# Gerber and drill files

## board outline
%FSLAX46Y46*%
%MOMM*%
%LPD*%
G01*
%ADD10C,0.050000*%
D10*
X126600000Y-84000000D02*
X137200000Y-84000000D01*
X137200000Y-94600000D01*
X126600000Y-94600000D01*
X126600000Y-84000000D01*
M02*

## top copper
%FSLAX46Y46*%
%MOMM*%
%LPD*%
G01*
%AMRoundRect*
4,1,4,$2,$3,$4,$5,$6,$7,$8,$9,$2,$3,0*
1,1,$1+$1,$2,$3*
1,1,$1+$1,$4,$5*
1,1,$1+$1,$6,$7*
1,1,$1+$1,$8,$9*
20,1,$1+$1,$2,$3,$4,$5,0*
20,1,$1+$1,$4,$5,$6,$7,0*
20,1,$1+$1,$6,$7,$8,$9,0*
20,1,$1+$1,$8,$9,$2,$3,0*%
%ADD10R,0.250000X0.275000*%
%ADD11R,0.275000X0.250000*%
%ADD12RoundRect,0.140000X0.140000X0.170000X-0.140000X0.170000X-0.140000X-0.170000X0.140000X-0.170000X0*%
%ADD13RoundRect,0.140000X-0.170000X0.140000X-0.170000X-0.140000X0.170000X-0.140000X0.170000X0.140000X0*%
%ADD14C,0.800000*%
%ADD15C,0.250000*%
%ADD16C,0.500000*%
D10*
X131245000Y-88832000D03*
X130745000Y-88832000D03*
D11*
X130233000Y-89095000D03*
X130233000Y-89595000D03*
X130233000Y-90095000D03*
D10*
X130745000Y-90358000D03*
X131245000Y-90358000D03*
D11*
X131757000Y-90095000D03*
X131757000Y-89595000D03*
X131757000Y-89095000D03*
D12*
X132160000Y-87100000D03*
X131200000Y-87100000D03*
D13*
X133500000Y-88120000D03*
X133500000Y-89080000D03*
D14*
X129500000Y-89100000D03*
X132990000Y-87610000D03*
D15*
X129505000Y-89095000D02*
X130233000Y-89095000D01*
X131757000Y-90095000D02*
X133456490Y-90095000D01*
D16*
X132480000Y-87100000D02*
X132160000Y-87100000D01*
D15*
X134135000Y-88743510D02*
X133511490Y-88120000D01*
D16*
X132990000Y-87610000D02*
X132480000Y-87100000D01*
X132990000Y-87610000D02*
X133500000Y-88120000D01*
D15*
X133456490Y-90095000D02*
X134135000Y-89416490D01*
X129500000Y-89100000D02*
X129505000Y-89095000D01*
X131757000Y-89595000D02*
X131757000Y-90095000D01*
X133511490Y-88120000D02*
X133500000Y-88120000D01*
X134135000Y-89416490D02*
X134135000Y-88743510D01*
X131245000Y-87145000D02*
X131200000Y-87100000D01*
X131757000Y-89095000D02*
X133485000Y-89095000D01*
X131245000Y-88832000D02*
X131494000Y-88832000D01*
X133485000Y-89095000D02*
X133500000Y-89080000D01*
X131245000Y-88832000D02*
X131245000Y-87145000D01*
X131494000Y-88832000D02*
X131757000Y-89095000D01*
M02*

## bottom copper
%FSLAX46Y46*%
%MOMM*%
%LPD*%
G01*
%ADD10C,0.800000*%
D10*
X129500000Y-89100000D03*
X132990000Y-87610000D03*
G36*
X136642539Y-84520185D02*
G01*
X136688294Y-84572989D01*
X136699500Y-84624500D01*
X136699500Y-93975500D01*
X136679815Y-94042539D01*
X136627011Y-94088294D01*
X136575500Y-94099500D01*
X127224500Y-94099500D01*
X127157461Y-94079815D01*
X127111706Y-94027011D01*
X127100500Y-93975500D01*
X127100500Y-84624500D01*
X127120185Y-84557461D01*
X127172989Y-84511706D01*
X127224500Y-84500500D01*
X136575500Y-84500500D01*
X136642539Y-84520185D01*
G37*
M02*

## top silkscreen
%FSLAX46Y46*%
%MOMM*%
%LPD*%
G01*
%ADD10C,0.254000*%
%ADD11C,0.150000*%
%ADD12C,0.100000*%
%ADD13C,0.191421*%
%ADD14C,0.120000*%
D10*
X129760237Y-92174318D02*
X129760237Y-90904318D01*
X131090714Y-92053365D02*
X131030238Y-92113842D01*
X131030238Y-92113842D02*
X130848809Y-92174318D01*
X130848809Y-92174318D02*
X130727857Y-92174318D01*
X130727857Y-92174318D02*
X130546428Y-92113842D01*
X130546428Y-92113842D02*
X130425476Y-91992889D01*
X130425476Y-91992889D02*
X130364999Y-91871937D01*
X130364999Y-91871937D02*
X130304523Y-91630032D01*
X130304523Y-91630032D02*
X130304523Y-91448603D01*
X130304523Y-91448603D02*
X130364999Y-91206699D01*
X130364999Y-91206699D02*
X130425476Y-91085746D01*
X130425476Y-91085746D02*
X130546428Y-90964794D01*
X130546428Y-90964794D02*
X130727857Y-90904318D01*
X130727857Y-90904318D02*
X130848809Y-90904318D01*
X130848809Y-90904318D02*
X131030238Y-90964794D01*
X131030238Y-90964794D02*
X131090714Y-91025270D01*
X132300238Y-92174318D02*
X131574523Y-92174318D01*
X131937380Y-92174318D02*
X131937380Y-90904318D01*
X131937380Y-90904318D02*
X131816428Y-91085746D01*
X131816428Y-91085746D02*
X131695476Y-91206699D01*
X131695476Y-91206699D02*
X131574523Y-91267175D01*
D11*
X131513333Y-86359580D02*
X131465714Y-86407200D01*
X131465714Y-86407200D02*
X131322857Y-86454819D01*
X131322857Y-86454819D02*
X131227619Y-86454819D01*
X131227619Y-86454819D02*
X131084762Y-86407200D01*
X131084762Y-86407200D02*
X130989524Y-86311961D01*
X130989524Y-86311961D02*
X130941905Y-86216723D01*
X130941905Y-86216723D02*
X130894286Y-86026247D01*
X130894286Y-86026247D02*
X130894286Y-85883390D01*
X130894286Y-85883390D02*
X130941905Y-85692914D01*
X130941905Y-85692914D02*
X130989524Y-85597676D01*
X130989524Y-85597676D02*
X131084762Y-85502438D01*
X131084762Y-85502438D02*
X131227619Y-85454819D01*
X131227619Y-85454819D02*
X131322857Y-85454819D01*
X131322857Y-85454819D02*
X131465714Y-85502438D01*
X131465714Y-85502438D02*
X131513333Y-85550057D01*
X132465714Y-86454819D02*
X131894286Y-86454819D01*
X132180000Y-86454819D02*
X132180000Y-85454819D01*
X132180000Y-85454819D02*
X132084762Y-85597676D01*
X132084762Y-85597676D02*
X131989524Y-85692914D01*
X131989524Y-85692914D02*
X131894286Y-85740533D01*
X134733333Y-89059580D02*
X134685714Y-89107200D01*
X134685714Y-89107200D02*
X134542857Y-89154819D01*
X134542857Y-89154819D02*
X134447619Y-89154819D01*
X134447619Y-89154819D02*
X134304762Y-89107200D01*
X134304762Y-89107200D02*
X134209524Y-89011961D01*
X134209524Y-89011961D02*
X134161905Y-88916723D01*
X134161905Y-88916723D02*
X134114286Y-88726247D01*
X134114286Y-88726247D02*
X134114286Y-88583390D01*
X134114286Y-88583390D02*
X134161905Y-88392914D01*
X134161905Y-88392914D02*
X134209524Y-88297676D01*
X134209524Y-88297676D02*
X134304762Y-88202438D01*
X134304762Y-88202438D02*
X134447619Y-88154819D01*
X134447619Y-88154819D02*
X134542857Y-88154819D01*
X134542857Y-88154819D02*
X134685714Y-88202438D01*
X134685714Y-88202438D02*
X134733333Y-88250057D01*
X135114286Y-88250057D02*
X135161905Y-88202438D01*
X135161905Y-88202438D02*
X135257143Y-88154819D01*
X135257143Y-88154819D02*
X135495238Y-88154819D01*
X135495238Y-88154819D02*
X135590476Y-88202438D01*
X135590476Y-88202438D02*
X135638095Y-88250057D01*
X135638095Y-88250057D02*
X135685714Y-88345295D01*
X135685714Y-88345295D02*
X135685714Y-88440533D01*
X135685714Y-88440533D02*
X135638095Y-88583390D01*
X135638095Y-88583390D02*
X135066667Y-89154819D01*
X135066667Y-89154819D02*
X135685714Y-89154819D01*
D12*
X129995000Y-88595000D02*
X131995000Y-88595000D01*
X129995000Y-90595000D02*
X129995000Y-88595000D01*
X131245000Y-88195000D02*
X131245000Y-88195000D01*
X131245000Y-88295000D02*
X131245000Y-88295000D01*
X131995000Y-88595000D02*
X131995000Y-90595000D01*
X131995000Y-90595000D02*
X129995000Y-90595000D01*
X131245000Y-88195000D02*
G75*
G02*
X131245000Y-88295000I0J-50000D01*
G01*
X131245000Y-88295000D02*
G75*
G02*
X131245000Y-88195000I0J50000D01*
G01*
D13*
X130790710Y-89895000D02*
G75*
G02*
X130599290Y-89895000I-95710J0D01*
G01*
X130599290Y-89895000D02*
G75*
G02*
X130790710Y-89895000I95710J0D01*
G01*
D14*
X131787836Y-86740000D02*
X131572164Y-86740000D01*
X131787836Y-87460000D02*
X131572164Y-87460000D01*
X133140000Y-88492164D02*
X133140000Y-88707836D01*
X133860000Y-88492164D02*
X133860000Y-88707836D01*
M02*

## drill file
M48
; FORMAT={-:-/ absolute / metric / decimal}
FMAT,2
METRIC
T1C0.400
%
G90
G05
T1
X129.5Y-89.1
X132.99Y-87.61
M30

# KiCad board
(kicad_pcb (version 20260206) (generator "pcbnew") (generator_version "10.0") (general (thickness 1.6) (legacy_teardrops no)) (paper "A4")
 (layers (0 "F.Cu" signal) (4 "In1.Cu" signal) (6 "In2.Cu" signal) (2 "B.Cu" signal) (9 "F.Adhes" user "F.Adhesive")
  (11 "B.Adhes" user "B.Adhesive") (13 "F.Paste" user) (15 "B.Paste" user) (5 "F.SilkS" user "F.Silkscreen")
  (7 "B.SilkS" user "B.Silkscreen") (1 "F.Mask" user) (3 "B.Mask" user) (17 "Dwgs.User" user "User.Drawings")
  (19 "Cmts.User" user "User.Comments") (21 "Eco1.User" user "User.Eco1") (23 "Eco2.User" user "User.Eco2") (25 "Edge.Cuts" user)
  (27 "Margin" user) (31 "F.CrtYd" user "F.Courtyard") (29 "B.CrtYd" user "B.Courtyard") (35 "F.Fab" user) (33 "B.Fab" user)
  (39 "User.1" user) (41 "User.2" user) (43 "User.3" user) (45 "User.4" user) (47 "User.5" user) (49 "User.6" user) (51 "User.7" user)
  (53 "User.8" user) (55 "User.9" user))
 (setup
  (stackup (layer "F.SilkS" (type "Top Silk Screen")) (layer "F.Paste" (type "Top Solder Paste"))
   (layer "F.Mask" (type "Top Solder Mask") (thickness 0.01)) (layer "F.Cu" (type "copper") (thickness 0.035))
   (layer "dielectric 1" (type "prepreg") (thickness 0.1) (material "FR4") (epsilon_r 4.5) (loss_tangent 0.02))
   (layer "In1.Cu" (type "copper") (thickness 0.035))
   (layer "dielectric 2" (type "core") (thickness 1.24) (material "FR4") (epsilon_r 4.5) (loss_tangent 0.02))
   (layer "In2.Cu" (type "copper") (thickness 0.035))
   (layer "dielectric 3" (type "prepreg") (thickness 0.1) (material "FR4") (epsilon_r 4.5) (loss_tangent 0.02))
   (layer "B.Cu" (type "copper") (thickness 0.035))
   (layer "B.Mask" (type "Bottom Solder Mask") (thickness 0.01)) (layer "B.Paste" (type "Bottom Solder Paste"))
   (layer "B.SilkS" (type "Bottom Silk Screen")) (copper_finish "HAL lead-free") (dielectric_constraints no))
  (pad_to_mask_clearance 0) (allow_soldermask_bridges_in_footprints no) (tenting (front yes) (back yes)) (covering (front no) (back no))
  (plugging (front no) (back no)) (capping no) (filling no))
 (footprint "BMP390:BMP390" (layer "F.Cu") (at 130.995 89.595)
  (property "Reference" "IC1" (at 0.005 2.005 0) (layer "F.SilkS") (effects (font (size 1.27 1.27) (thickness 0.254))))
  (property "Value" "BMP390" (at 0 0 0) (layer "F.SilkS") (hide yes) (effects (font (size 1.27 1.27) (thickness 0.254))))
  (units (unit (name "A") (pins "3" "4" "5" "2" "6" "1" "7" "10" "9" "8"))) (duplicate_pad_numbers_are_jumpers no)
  (fp_line (start -1 -1) (end 1 -1) (stroke (width 0.1) (type solid)) (layer "F.SilkS"))
  (fp_line (start -1 1) (end -1 -1) (stroke (width 0.1) (type solid)) (layer "F.SilkS"))
  (fp_line (start 0.25 -1.4) (end 0.25 -1.4) (stroke (width 0.1) (type solid)) (layer "F.SilkS"))
  (fp_line (start 0.25 -1.3) (end 0.25 -1.3) (stroke (width 0.1) (type solid)) (layer "F.SilkS"))
  (fp_line (start 1 -1) (end 1 1) (stroke (width 0.1) (type solid)) (layer "F.SilkS"))
  (fp_line (start 1 1) (end -1 1) (stroke (width 0.1) (type solid)) (layer "F.SilkS"))
  (fp_arc (start 0.25 -1.4) (mid 0.3 -1.35) (end 0.25 -1.3) (stroke (width 0.1) (type solid)) (layer "F.SilkS"))
  (fp_arc (start 0.25 -1.3) (mid 0.2 -1.35) (end 0.25 -1.4) (stroke (width 0.1) (type solid)) (layer "F.SilkS"))
  (fp_circle (center -0.3 0.3) (end -0.4 0.2) (stroke (width 0.1) (type solid)) (fill yes) (layer "F.SilkS"))
  (pad "1" smd rect (at 0.25 -0.763) (size 0.25 0.275) (layers "F.Cu" "F.Mask" "F.Paste") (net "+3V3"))
  (pad "2" smd rect (at -0.25 -0.763) (size 0.25 0.275) (layers "F.Cu" "F.Mask" "F.Paste") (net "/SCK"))
  (pad "3" smd rect (at -0.762 -0.5 90) (size 0.25 0.275) (layers "F.Cu" "F.Mask" "F.Paste") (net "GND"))
  (pad "4" smd rect (at -0.762 0 90) (size 0.25 0.275) (layers "F.Cu" "F.Mask" "F.Paste") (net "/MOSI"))
  (pad "5" smd rect (at -0.762 0.5 90) (size 0.25 0.275) (layers "F.Cu" "F.Mask" "F.Paste") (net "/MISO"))
  (pad "6" smd rect (at -0.25 0.763) (size 0.25 0.275) (layers "F.Cu" "F.Mask" "F.Paste") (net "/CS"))
  (pad "7" smd rect (at 0.25 0.763) (size 0.25 0.275) (layers "F.Cu" "F.Mask" "F.Paste") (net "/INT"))
  (pad "8" smd rect (at 0.762 0.5 90) (size 0.25 0.275) (layers "F.Cu" "F.Mask" "F.Paste") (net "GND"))
  (pad "9" smd rect (at 0.762 0 90) (size 0.25 0.275) (layers "F.Cu" "F.Mask" "F.Paste") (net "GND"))
  (pad "10" smd rect (at 0.762 -0.5 90) (size 0.25 0.275) (layers "F.Cu" "F.Mask" "F.Paste") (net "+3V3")))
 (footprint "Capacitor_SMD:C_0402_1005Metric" (layer "F.Cu") (at 131.68 87.1 180)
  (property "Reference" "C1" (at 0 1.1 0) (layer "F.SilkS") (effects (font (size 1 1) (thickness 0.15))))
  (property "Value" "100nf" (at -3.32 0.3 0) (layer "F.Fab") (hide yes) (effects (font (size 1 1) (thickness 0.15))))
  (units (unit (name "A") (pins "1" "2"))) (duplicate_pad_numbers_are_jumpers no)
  (fp_line (start -0.107836 0.36) (end 0.107836 0.36) (stroke (width 0.12) (type solid)) (layer "F.SilkS"))
  (fp_line (start -0.107836 -0.36) (end 0.107836 -0.36) (stroke (width 0.12) (type solid)) (layer "F.SilkS"))
  (pad "1" smd roundrect (at -0.48 0 180) (size 0.56 0.62) (layers "F.Cu" "F.Mask" "F.Paste") (roundrect_rratio 0.25) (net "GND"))
  (pad "2" smd roundrect (at 0.48 0 180) (size 0.56 0.62) (layers "F.Cu" "F.Mask" "F.Paste") (roundrect_rratio 0.25) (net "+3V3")))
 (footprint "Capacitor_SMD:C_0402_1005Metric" (layer "F.Cu") (at 133.5 88.6 -90)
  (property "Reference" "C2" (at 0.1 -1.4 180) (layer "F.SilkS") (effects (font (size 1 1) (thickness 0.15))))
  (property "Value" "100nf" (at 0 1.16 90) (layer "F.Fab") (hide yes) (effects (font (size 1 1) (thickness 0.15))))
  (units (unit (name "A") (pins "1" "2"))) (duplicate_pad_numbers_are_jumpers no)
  (fp_line (start -0.107836 0.36) (end 0.107836 0.36) (stroke (width 0.12) (type solid)) (layer "F.SilkS"))
  (fp_line (start -0.107836 -0.36) (end 0.107836 -0.36) (stroke (width 0.12) (type solid)) (layer "F.SilkS"))
  (pad "1" smd roundrect (at -0.48 0 270) (size 0.56 0.62) (layers "F.Cu" "F.Mask" "F.Paste") (roundrect_rratio 0.25) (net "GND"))
  (pad "2" smd roundrect (at 0.48 0 270) (size 0.56 0.62) (layers "F.Cu" "F.Mask" "F.Paste") (roundrect_rratio 0.25) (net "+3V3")))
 (gr_rect (start 126.6 84) (end 137.2 94.6) (stroke (width 0.05) (type default)) (fill no) (layer "Edge.Cuts"))
 (segment (start 129.505 89.095) (end 130.233 89.095) (width 0.25) (layer "F.Cu") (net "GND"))
 (segment (start 131.757 90.095) (end 133.45649 90.095) (width 0.25) (layer "F.Cu") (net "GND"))
 (segment (start 132.48 87.1) (end 132.16 87.1) (width 0.5) (layer "F.Cu") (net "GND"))
 (segment (start 134.135 88.74351) (end 133.51149 88.12) (width 0.25) (layer "F.Cu") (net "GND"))
 (segment (start 132.99 87.61) (end 132.48 87.1) (width 0.5) (layer "F.Cu") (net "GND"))
 (segment (start 132.99 87.61) (end 133.5 88.12) (width 0.5) (layer "F.Cu") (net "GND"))
 (segment (start 133.45649 90.095) (end 134.135 89.41649) (width 0.25) (layer "F.Cu") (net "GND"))
 (segment (start 129.5 89.1) (end 129.505 89.095) (width 0.25) (layer "F.Cu") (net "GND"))
 (segment (start 131.757 89.595) (end 131.757 90.095) (width 0.25) (layer "F.Cu") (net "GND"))
 (segment (start 133.51149 88.12) (end 133.5 88.12) (width 0.25) (layer "F.Cu") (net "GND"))
 (segment (start 134.135 89.41649) (end 134.135 88.74351) (width 0.25) (layer "F.Cu") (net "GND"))
 (via (at 129.5 89.1) (size 0.8) (drill 0.4) (layers "F.Cu" "B.Cu") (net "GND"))
 (via (at 132.99 87.61) (size 0.8) (drill 0.4) (layers "F.Cu" "B.Cu") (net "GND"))
 (segment (start 131.245 87.145) (end 131.2 87.1) (width 0.25) (layer "F.Cu") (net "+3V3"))
 (segment (start 131.757 89.095) (end 133.485 89.095) (width 0.25) (layer "F.Cu") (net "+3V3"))
 (segment (start 131.245 88.832) (end 131.494 88.832) (width 0.25) (layer "F.Cu") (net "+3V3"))
 (segment (start 133.485 89.095) (end 133.5 89.08) (width 0.25) (layer "F.Cu") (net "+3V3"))
 (segment (start 131.245 88.832) (end 131.245 87.145) (width 0.25) (layer "F.Cu") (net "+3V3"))
 (segment (start 131.494 88.832) (end 131.757 89.095) (width 0.25) (layer "F.Cu") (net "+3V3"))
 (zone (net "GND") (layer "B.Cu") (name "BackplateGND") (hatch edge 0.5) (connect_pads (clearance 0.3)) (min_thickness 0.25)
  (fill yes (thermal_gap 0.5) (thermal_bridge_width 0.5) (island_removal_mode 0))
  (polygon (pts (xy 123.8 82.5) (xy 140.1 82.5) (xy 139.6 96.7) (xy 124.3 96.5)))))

